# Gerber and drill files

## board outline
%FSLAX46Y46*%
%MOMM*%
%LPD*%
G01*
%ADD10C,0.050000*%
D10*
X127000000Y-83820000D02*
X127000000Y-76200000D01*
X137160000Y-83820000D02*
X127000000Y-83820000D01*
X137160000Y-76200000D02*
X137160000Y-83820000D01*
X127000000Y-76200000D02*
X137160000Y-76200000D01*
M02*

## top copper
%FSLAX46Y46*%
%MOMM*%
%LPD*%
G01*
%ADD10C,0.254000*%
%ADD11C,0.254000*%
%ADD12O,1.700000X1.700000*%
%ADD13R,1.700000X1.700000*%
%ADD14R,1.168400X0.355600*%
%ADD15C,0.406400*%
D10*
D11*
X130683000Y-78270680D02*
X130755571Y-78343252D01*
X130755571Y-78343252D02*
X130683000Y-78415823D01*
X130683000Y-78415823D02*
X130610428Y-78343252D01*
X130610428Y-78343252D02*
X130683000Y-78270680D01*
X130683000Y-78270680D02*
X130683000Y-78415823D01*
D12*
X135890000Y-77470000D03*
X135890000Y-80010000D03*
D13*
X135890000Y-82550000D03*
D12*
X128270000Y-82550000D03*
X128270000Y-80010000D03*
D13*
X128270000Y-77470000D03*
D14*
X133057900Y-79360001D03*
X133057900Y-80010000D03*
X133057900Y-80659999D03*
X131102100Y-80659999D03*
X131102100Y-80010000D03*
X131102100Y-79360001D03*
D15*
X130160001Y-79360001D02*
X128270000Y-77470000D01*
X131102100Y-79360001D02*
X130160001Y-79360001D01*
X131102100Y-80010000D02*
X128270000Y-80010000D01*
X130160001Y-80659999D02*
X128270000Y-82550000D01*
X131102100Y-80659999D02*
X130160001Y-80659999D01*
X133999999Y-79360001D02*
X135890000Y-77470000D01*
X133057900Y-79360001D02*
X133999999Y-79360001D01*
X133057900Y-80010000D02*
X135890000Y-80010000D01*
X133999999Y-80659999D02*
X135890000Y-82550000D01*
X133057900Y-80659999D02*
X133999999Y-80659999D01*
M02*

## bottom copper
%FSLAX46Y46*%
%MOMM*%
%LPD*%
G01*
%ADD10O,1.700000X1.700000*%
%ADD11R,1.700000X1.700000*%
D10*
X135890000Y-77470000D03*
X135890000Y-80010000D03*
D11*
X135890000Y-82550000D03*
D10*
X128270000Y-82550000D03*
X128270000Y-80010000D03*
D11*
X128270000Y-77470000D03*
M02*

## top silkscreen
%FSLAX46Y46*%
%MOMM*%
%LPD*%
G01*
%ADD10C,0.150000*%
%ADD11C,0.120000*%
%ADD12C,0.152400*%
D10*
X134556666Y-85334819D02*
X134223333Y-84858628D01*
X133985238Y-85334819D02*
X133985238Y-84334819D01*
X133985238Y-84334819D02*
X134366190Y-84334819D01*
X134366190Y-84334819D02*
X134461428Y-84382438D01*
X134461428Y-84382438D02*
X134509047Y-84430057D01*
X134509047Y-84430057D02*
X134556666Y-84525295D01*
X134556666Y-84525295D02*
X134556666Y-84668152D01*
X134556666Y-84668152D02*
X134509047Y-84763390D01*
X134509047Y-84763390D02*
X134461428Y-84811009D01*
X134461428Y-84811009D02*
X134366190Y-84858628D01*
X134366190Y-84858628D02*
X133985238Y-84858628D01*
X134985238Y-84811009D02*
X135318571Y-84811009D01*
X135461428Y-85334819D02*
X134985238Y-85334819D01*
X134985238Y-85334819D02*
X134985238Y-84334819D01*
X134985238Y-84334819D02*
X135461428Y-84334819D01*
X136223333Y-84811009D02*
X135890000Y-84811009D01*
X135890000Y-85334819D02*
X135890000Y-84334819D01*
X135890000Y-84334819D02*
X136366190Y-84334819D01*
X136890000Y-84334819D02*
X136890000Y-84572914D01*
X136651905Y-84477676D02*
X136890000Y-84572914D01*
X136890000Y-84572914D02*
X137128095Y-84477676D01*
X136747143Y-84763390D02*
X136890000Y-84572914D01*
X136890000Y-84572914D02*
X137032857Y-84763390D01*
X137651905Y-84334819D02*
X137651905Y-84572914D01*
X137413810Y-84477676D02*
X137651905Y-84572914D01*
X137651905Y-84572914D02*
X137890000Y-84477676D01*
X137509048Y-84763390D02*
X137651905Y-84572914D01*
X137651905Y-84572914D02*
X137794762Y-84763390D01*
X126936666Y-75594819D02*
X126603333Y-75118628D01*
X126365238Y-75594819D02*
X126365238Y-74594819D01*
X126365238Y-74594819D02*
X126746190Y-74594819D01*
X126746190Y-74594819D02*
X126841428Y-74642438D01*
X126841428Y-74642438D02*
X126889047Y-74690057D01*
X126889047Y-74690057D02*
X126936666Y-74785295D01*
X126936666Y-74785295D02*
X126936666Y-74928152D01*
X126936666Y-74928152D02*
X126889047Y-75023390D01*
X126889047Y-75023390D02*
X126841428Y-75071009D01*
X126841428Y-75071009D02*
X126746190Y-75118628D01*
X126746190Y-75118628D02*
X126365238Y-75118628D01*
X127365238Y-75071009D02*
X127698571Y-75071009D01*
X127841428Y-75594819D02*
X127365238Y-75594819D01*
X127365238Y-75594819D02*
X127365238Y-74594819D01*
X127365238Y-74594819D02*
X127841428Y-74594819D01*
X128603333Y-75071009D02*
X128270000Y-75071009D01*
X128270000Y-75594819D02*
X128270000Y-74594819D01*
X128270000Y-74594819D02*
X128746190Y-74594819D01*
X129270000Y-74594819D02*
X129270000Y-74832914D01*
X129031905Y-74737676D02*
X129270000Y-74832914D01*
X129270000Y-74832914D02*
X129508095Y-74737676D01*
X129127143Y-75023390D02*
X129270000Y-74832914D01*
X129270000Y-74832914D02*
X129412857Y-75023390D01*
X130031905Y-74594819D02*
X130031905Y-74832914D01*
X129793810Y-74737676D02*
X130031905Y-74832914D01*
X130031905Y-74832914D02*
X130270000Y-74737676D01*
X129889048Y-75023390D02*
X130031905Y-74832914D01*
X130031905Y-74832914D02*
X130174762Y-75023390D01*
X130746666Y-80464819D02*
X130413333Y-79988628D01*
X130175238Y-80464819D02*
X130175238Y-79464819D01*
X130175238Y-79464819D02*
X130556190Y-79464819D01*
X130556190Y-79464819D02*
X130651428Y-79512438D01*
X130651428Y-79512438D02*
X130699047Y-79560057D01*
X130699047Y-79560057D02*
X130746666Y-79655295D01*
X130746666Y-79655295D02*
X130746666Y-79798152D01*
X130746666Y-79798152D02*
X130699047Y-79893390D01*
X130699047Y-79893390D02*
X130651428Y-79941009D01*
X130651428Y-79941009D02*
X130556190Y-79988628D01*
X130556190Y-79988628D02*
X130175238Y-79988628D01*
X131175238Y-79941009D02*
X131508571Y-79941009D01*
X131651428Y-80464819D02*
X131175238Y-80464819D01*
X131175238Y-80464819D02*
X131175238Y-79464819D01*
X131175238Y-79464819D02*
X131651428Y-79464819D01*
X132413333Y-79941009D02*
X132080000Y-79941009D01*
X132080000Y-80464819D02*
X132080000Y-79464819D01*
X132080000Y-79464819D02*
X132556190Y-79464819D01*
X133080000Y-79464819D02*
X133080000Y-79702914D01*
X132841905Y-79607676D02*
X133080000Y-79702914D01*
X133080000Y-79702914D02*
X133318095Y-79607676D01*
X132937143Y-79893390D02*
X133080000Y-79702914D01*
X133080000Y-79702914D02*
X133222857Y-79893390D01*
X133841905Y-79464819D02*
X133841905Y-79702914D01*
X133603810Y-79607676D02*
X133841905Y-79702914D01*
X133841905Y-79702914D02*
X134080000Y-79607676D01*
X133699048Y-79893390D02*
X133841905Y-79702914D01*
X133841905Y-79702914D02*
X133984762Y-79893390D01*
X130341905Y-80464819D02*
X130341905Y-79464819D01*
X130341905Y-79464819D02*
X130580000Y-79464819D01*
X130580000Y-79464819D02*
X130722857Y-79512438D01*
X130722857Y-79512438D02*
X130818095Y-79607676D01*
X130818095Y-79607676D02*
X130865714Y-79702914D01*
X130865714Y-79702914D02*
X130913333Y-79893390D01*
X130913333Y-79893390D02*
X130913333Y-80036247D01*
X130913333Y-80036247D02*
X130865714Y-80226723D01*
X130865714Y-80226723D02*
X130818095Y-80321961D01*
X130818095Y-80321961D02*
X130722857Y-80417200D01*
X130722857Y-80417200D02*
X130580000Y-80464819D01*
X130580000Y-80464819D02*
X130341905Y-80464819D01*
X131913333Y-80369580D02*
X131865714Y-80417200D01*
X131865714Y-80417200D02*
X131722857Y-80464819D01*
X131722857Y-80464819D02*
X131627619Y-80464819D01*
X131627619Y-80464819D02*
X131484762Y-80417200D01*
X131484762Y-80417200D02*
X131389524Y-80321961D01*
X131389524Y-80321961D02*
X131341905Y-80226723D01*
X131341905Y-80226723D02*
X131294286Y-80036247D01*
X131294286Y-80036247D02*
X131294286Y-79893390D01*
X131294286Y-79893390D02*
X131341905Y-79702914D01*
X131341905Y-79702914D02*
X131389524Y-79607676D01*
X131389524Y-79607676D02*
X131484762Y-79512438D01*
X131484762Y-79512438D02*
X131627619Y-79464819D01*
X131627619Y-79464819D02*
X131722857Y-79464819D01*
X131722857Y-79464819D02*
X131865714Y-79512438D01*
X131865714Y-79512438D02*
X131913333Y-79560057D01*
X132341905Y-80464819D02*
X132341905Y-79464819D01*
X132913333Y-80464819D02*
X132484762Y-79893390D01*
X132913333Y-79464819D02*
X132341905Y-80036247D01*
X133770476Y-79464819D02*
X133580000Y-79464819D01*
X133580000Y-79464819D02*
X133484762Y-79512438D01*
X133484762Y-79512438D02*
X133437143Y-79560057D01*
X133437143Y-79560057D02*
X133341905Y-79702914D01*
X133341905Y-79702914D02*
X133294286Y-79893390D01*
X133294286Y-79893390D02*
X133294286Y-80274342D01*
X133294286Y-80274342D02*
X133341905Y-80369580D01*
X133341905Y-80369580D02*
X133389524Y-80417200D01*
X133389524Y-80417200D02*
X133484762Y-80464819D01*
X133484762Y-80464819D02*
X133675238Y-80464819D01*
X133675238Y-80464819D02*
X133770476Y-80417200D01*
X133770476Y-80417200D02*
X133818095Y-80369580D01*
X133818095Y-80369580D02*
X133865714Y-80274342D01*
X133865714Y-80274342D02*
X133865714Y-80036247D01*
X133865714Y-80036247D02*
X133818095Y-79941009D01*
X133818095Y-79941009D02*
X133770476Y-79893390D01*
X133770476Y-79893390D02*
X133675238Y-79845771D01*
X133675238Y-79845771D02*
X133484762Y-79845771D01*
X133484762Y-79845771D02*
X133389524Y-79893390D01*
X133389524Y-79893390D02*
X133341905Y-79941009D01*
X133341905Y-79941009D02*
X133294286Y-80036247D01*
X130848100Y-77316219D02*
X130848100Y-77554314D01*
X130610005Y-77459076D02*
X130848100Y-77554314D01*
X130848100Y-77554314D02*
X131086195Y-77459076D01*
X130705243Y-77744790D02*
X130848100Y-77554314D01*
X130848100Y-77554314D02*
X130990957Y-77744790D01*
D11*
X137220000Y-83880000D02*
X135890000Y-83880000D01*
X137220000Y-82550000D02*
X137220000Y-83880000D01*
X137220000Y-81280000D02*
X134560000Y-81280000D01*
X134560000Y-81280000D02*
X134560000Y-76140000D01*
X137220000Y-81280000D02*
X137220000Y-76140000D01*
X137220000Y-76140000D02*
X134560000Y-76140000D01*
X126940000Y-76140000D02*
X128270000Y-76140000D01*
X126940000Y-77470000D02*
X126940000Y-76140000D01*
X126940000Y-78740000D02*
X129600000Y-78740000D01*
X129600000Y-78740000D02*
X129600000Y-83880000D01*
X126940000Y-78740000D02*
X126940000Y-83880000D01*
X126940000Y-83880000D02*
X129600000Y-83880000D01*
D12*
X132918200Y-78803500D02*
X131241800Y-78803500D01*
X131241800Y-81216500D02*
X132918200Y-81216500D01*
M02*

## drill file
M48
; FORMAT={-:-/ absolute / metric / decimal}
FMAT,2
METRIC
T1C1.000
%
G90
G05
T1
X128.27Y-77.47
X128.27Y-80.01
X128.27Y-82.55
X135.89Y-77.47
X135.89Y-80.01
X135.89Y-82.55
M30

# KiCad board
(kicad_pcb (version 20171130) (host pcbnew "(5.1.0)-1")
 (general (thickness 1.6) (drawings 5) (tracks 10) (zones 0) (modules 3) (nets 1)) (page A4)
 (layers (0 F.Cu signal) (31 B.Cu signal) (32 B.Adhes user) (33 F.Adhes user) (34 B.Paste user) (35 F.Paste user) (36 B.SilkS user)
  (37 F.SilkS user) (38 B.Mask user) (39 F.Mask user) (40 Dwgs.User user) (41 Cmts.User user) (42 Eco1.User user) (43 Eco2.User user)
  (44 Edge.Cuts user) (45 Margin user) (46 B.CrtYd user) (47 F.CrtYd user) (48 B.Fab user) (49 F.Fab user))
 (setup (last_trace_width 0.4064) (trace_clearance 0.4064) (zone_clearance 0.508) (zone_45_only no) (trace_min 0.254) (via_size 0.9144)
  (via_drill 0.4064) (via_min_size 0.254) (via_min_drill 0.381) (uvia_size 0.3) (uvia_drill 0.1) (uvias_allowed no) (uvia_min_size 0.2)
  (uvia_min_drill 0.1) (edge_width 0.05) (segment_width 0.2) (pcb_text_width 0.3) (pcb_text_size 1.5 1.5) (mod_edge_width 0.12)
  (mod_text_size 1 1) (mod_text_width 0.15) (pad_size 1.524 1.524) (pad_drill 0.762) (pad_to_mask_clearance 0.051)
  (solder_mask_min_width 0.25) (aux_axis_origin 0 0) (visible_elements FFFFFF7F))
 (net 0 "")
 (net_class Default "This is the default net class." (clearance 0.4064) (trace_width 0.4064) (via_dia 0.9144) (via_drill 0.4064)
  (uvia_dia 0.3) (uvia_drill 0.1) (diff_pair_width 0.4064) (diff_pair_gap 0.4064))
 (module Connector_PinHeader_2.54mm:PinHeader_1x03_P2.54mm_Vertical (layer F.Cu) (at 135.89 82.55 180)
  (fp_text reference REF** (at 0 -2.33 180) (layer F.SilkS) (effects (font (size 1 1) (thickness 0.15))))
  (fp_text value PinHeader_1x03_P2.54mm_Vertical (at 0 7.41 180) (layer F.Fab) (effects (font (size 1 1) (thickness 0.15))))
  (fp_line (start -1.33 -1.33) (end 0 -1.33) (layer F.SilkS) (width 0.12))
  (fp_line (start -1.33 0) (end -1.33 -1.33) (layer F.SilkS) (width 0.12))
  (fp_line (start -1.33 1.27) (end 1.33 1.27) (layer F.SilkS) (width 0.12))
  (fp_line (start 1.33 1.27) (end 1.33 6.41) (layer F.SilkS) (width 0.12))
  (fp_line (start -1.33 1.27) (end -1.33 6.41) (layer F.SilkS) (width 0.12))
  (fp_line (start -1.33 6.41) (end 1.33 6.41) (layer F.SilkS) (width 0.12))
  (pad 3 thru_hole oval (at 0 5.08 180) (size 1.7 1.7) (drill 1) (layers *.Cu *.Mask))
  (pad 2 thru_hole oval (at 0 2.54 180) (size 1.7 1.7) (drill 1) (layers *.Cu *.Mask))
  (pad 1 thru_hole rect (at 0 0 180) (size 1.7 1.7) (drill 1) (layers *.Cu *.Mask)))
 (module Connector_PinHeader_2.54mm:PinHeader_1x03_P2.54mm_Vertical (layer F.Cu) (at 128.27 77.47)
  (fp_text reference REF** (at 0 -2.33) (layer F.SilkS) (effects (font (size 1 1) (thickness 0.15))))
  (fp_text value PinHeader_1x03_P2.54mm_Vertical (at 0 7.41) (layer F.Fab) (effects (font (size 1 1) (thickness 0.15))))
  (fp_line (start -1.33 -1.33) (end 0 -1.33) (layer F.SilkS) (width 0.12))
  (fp_line (start -1.33 0) (end -1.33 -1.33) (layer F.SilkS) (width 0.12))
  (fp_line (start -1.33 1.27) (end 1.33 1.27) (layer F.SilkS) (width 0.12))
  (fp_line (start 1.33 1.27) (end 1.33 6.41) (layer F.SilkS) (width 0.12))
  (fp_line (start -1.33 1.27) (end -1.33 6.41) (layer F.SilkS) (width 0.12))
  (fp_line (start -1.33 6.41) (end 1.33 6.41) (layer F.SilkS) (width 0.12))
  (pad 3 thru_hole oval (at 0 5.08) (size 1.7 1.7) (drill 1) (layers *.Cu *.Mask))
  (pad 2 thru_hole oval (at 0 2.54) (size 1.7 1.7) (drill 1) (layers *.Cu *.Mask))
  (pad 1 thru_hole rect (at 0 0) (size 1.7 1.7) (drill 1) (layers *.Cu *.Mask)))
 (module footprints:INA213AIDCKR (layer F.Cu) (at 132.08 80.01)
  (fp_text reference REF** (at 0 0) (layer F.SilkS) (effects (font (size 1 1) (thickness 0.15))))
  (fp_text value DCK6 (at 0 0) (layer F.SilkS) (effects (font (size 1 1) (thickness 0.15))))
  (fp_line (start 0.8382 -1.2065) (end -0.8382 -1.2065) (layer F.SilkS) (width 0.1524))
  (fp_line (start -0.8382 1.2065) (end 0.8382 1.2065) (layer F.SilkS) (width 0.1524))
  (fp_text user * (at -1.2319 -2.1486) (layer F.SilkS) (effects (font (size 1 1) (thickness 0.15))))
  (pad 6 smd rect (at 0.9779 -0.649999) (size 1.1684 0.3556) (layers F.Cu F.Paste F.Mask))
  (pad 5 smd rect (at 0.9779 0) (size 1.1684 0.3556) (layers F.Cu F.Paste F.Mask))
  (pad 4 smd rect (at 0.9779 0.649999) (size 1.1684 0.3556) (layers F.Cu F.Paste F.Mask))
  (pad 3 smd rect (at -0.9779 0.649999) (size 1.1684 0.3556) (layers F.Cu F.Paste F.Mask))
  (pad 2 smd rect (at -0.9779 0) (size 1.1684 0.3556) (layers F.Cu F.Paste F.Mask))
  (pad 1 smd rect (at -0.9779 -0.649999) (size 1.1684 0.3556) (layers F.Cu F.Paste F.Mask)))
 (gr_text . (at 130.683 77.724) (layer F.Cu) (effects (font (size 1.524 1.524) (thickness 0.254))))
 (gr_line (start 127 83.82) (end 127 76.2) (layer Edge.Cuts) (width 0.05))
 (gr_line (start 137.16 83.82) (end 127 83.82) (layer Edge.Cuts) (width 0.05))
 (gr_line (start 137.16 76.2) (end 137.16 83.82) (layer Edge.Cuts) (width 0.05))
 (gr_line (start 127 76.2) (end 137.16 76.2) (layer Edge.Cuts) (width 0.05))
 (segment (start 130.160001 79.360001) (end 128.27 77.47) (width 0.4064) (layer F.Cu) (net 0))
 (segment (start 131.1021 79.360001) (end 130.160001 79.360001) (width 0.4064) (layer F.Cu) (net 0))
 (segment (start 131.1021 80.01) (end 128.27 80.01) (width 0.4064) (layer F.Cu) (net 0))
 (segment (start 130.160001 80.659999) (end 128.27 82.55) (width 0.4064) (layer F.Cu) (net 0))
 (segment (start 131.1021 80.659999) (end 130.160001 80.659999) (width 0.4064) (layer F.Cu) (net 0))
 (segment (start 133.999999 79.360001) (end 135.89 77.47) (width 0.4064) (layer F.Cu) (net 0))
 (segment (start 133.0579 79.360001) (end 133.999999 79.360001) (width 0.4064) (layer F.Cu) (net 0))
 (segment (start 133.0579 80.01) (end 135.89 80.01) (width 0.4064) (layer F.Cu) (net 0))
 (segment (start 133.999999 80.659999) (end 135.89 82.55) (width 0.4064) (layer F.Cu) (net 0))
 (segment (start 133.0579 80.659999) (end 133.999999 80.659999) (width 0.4064) (layer F.Cu) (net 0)))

